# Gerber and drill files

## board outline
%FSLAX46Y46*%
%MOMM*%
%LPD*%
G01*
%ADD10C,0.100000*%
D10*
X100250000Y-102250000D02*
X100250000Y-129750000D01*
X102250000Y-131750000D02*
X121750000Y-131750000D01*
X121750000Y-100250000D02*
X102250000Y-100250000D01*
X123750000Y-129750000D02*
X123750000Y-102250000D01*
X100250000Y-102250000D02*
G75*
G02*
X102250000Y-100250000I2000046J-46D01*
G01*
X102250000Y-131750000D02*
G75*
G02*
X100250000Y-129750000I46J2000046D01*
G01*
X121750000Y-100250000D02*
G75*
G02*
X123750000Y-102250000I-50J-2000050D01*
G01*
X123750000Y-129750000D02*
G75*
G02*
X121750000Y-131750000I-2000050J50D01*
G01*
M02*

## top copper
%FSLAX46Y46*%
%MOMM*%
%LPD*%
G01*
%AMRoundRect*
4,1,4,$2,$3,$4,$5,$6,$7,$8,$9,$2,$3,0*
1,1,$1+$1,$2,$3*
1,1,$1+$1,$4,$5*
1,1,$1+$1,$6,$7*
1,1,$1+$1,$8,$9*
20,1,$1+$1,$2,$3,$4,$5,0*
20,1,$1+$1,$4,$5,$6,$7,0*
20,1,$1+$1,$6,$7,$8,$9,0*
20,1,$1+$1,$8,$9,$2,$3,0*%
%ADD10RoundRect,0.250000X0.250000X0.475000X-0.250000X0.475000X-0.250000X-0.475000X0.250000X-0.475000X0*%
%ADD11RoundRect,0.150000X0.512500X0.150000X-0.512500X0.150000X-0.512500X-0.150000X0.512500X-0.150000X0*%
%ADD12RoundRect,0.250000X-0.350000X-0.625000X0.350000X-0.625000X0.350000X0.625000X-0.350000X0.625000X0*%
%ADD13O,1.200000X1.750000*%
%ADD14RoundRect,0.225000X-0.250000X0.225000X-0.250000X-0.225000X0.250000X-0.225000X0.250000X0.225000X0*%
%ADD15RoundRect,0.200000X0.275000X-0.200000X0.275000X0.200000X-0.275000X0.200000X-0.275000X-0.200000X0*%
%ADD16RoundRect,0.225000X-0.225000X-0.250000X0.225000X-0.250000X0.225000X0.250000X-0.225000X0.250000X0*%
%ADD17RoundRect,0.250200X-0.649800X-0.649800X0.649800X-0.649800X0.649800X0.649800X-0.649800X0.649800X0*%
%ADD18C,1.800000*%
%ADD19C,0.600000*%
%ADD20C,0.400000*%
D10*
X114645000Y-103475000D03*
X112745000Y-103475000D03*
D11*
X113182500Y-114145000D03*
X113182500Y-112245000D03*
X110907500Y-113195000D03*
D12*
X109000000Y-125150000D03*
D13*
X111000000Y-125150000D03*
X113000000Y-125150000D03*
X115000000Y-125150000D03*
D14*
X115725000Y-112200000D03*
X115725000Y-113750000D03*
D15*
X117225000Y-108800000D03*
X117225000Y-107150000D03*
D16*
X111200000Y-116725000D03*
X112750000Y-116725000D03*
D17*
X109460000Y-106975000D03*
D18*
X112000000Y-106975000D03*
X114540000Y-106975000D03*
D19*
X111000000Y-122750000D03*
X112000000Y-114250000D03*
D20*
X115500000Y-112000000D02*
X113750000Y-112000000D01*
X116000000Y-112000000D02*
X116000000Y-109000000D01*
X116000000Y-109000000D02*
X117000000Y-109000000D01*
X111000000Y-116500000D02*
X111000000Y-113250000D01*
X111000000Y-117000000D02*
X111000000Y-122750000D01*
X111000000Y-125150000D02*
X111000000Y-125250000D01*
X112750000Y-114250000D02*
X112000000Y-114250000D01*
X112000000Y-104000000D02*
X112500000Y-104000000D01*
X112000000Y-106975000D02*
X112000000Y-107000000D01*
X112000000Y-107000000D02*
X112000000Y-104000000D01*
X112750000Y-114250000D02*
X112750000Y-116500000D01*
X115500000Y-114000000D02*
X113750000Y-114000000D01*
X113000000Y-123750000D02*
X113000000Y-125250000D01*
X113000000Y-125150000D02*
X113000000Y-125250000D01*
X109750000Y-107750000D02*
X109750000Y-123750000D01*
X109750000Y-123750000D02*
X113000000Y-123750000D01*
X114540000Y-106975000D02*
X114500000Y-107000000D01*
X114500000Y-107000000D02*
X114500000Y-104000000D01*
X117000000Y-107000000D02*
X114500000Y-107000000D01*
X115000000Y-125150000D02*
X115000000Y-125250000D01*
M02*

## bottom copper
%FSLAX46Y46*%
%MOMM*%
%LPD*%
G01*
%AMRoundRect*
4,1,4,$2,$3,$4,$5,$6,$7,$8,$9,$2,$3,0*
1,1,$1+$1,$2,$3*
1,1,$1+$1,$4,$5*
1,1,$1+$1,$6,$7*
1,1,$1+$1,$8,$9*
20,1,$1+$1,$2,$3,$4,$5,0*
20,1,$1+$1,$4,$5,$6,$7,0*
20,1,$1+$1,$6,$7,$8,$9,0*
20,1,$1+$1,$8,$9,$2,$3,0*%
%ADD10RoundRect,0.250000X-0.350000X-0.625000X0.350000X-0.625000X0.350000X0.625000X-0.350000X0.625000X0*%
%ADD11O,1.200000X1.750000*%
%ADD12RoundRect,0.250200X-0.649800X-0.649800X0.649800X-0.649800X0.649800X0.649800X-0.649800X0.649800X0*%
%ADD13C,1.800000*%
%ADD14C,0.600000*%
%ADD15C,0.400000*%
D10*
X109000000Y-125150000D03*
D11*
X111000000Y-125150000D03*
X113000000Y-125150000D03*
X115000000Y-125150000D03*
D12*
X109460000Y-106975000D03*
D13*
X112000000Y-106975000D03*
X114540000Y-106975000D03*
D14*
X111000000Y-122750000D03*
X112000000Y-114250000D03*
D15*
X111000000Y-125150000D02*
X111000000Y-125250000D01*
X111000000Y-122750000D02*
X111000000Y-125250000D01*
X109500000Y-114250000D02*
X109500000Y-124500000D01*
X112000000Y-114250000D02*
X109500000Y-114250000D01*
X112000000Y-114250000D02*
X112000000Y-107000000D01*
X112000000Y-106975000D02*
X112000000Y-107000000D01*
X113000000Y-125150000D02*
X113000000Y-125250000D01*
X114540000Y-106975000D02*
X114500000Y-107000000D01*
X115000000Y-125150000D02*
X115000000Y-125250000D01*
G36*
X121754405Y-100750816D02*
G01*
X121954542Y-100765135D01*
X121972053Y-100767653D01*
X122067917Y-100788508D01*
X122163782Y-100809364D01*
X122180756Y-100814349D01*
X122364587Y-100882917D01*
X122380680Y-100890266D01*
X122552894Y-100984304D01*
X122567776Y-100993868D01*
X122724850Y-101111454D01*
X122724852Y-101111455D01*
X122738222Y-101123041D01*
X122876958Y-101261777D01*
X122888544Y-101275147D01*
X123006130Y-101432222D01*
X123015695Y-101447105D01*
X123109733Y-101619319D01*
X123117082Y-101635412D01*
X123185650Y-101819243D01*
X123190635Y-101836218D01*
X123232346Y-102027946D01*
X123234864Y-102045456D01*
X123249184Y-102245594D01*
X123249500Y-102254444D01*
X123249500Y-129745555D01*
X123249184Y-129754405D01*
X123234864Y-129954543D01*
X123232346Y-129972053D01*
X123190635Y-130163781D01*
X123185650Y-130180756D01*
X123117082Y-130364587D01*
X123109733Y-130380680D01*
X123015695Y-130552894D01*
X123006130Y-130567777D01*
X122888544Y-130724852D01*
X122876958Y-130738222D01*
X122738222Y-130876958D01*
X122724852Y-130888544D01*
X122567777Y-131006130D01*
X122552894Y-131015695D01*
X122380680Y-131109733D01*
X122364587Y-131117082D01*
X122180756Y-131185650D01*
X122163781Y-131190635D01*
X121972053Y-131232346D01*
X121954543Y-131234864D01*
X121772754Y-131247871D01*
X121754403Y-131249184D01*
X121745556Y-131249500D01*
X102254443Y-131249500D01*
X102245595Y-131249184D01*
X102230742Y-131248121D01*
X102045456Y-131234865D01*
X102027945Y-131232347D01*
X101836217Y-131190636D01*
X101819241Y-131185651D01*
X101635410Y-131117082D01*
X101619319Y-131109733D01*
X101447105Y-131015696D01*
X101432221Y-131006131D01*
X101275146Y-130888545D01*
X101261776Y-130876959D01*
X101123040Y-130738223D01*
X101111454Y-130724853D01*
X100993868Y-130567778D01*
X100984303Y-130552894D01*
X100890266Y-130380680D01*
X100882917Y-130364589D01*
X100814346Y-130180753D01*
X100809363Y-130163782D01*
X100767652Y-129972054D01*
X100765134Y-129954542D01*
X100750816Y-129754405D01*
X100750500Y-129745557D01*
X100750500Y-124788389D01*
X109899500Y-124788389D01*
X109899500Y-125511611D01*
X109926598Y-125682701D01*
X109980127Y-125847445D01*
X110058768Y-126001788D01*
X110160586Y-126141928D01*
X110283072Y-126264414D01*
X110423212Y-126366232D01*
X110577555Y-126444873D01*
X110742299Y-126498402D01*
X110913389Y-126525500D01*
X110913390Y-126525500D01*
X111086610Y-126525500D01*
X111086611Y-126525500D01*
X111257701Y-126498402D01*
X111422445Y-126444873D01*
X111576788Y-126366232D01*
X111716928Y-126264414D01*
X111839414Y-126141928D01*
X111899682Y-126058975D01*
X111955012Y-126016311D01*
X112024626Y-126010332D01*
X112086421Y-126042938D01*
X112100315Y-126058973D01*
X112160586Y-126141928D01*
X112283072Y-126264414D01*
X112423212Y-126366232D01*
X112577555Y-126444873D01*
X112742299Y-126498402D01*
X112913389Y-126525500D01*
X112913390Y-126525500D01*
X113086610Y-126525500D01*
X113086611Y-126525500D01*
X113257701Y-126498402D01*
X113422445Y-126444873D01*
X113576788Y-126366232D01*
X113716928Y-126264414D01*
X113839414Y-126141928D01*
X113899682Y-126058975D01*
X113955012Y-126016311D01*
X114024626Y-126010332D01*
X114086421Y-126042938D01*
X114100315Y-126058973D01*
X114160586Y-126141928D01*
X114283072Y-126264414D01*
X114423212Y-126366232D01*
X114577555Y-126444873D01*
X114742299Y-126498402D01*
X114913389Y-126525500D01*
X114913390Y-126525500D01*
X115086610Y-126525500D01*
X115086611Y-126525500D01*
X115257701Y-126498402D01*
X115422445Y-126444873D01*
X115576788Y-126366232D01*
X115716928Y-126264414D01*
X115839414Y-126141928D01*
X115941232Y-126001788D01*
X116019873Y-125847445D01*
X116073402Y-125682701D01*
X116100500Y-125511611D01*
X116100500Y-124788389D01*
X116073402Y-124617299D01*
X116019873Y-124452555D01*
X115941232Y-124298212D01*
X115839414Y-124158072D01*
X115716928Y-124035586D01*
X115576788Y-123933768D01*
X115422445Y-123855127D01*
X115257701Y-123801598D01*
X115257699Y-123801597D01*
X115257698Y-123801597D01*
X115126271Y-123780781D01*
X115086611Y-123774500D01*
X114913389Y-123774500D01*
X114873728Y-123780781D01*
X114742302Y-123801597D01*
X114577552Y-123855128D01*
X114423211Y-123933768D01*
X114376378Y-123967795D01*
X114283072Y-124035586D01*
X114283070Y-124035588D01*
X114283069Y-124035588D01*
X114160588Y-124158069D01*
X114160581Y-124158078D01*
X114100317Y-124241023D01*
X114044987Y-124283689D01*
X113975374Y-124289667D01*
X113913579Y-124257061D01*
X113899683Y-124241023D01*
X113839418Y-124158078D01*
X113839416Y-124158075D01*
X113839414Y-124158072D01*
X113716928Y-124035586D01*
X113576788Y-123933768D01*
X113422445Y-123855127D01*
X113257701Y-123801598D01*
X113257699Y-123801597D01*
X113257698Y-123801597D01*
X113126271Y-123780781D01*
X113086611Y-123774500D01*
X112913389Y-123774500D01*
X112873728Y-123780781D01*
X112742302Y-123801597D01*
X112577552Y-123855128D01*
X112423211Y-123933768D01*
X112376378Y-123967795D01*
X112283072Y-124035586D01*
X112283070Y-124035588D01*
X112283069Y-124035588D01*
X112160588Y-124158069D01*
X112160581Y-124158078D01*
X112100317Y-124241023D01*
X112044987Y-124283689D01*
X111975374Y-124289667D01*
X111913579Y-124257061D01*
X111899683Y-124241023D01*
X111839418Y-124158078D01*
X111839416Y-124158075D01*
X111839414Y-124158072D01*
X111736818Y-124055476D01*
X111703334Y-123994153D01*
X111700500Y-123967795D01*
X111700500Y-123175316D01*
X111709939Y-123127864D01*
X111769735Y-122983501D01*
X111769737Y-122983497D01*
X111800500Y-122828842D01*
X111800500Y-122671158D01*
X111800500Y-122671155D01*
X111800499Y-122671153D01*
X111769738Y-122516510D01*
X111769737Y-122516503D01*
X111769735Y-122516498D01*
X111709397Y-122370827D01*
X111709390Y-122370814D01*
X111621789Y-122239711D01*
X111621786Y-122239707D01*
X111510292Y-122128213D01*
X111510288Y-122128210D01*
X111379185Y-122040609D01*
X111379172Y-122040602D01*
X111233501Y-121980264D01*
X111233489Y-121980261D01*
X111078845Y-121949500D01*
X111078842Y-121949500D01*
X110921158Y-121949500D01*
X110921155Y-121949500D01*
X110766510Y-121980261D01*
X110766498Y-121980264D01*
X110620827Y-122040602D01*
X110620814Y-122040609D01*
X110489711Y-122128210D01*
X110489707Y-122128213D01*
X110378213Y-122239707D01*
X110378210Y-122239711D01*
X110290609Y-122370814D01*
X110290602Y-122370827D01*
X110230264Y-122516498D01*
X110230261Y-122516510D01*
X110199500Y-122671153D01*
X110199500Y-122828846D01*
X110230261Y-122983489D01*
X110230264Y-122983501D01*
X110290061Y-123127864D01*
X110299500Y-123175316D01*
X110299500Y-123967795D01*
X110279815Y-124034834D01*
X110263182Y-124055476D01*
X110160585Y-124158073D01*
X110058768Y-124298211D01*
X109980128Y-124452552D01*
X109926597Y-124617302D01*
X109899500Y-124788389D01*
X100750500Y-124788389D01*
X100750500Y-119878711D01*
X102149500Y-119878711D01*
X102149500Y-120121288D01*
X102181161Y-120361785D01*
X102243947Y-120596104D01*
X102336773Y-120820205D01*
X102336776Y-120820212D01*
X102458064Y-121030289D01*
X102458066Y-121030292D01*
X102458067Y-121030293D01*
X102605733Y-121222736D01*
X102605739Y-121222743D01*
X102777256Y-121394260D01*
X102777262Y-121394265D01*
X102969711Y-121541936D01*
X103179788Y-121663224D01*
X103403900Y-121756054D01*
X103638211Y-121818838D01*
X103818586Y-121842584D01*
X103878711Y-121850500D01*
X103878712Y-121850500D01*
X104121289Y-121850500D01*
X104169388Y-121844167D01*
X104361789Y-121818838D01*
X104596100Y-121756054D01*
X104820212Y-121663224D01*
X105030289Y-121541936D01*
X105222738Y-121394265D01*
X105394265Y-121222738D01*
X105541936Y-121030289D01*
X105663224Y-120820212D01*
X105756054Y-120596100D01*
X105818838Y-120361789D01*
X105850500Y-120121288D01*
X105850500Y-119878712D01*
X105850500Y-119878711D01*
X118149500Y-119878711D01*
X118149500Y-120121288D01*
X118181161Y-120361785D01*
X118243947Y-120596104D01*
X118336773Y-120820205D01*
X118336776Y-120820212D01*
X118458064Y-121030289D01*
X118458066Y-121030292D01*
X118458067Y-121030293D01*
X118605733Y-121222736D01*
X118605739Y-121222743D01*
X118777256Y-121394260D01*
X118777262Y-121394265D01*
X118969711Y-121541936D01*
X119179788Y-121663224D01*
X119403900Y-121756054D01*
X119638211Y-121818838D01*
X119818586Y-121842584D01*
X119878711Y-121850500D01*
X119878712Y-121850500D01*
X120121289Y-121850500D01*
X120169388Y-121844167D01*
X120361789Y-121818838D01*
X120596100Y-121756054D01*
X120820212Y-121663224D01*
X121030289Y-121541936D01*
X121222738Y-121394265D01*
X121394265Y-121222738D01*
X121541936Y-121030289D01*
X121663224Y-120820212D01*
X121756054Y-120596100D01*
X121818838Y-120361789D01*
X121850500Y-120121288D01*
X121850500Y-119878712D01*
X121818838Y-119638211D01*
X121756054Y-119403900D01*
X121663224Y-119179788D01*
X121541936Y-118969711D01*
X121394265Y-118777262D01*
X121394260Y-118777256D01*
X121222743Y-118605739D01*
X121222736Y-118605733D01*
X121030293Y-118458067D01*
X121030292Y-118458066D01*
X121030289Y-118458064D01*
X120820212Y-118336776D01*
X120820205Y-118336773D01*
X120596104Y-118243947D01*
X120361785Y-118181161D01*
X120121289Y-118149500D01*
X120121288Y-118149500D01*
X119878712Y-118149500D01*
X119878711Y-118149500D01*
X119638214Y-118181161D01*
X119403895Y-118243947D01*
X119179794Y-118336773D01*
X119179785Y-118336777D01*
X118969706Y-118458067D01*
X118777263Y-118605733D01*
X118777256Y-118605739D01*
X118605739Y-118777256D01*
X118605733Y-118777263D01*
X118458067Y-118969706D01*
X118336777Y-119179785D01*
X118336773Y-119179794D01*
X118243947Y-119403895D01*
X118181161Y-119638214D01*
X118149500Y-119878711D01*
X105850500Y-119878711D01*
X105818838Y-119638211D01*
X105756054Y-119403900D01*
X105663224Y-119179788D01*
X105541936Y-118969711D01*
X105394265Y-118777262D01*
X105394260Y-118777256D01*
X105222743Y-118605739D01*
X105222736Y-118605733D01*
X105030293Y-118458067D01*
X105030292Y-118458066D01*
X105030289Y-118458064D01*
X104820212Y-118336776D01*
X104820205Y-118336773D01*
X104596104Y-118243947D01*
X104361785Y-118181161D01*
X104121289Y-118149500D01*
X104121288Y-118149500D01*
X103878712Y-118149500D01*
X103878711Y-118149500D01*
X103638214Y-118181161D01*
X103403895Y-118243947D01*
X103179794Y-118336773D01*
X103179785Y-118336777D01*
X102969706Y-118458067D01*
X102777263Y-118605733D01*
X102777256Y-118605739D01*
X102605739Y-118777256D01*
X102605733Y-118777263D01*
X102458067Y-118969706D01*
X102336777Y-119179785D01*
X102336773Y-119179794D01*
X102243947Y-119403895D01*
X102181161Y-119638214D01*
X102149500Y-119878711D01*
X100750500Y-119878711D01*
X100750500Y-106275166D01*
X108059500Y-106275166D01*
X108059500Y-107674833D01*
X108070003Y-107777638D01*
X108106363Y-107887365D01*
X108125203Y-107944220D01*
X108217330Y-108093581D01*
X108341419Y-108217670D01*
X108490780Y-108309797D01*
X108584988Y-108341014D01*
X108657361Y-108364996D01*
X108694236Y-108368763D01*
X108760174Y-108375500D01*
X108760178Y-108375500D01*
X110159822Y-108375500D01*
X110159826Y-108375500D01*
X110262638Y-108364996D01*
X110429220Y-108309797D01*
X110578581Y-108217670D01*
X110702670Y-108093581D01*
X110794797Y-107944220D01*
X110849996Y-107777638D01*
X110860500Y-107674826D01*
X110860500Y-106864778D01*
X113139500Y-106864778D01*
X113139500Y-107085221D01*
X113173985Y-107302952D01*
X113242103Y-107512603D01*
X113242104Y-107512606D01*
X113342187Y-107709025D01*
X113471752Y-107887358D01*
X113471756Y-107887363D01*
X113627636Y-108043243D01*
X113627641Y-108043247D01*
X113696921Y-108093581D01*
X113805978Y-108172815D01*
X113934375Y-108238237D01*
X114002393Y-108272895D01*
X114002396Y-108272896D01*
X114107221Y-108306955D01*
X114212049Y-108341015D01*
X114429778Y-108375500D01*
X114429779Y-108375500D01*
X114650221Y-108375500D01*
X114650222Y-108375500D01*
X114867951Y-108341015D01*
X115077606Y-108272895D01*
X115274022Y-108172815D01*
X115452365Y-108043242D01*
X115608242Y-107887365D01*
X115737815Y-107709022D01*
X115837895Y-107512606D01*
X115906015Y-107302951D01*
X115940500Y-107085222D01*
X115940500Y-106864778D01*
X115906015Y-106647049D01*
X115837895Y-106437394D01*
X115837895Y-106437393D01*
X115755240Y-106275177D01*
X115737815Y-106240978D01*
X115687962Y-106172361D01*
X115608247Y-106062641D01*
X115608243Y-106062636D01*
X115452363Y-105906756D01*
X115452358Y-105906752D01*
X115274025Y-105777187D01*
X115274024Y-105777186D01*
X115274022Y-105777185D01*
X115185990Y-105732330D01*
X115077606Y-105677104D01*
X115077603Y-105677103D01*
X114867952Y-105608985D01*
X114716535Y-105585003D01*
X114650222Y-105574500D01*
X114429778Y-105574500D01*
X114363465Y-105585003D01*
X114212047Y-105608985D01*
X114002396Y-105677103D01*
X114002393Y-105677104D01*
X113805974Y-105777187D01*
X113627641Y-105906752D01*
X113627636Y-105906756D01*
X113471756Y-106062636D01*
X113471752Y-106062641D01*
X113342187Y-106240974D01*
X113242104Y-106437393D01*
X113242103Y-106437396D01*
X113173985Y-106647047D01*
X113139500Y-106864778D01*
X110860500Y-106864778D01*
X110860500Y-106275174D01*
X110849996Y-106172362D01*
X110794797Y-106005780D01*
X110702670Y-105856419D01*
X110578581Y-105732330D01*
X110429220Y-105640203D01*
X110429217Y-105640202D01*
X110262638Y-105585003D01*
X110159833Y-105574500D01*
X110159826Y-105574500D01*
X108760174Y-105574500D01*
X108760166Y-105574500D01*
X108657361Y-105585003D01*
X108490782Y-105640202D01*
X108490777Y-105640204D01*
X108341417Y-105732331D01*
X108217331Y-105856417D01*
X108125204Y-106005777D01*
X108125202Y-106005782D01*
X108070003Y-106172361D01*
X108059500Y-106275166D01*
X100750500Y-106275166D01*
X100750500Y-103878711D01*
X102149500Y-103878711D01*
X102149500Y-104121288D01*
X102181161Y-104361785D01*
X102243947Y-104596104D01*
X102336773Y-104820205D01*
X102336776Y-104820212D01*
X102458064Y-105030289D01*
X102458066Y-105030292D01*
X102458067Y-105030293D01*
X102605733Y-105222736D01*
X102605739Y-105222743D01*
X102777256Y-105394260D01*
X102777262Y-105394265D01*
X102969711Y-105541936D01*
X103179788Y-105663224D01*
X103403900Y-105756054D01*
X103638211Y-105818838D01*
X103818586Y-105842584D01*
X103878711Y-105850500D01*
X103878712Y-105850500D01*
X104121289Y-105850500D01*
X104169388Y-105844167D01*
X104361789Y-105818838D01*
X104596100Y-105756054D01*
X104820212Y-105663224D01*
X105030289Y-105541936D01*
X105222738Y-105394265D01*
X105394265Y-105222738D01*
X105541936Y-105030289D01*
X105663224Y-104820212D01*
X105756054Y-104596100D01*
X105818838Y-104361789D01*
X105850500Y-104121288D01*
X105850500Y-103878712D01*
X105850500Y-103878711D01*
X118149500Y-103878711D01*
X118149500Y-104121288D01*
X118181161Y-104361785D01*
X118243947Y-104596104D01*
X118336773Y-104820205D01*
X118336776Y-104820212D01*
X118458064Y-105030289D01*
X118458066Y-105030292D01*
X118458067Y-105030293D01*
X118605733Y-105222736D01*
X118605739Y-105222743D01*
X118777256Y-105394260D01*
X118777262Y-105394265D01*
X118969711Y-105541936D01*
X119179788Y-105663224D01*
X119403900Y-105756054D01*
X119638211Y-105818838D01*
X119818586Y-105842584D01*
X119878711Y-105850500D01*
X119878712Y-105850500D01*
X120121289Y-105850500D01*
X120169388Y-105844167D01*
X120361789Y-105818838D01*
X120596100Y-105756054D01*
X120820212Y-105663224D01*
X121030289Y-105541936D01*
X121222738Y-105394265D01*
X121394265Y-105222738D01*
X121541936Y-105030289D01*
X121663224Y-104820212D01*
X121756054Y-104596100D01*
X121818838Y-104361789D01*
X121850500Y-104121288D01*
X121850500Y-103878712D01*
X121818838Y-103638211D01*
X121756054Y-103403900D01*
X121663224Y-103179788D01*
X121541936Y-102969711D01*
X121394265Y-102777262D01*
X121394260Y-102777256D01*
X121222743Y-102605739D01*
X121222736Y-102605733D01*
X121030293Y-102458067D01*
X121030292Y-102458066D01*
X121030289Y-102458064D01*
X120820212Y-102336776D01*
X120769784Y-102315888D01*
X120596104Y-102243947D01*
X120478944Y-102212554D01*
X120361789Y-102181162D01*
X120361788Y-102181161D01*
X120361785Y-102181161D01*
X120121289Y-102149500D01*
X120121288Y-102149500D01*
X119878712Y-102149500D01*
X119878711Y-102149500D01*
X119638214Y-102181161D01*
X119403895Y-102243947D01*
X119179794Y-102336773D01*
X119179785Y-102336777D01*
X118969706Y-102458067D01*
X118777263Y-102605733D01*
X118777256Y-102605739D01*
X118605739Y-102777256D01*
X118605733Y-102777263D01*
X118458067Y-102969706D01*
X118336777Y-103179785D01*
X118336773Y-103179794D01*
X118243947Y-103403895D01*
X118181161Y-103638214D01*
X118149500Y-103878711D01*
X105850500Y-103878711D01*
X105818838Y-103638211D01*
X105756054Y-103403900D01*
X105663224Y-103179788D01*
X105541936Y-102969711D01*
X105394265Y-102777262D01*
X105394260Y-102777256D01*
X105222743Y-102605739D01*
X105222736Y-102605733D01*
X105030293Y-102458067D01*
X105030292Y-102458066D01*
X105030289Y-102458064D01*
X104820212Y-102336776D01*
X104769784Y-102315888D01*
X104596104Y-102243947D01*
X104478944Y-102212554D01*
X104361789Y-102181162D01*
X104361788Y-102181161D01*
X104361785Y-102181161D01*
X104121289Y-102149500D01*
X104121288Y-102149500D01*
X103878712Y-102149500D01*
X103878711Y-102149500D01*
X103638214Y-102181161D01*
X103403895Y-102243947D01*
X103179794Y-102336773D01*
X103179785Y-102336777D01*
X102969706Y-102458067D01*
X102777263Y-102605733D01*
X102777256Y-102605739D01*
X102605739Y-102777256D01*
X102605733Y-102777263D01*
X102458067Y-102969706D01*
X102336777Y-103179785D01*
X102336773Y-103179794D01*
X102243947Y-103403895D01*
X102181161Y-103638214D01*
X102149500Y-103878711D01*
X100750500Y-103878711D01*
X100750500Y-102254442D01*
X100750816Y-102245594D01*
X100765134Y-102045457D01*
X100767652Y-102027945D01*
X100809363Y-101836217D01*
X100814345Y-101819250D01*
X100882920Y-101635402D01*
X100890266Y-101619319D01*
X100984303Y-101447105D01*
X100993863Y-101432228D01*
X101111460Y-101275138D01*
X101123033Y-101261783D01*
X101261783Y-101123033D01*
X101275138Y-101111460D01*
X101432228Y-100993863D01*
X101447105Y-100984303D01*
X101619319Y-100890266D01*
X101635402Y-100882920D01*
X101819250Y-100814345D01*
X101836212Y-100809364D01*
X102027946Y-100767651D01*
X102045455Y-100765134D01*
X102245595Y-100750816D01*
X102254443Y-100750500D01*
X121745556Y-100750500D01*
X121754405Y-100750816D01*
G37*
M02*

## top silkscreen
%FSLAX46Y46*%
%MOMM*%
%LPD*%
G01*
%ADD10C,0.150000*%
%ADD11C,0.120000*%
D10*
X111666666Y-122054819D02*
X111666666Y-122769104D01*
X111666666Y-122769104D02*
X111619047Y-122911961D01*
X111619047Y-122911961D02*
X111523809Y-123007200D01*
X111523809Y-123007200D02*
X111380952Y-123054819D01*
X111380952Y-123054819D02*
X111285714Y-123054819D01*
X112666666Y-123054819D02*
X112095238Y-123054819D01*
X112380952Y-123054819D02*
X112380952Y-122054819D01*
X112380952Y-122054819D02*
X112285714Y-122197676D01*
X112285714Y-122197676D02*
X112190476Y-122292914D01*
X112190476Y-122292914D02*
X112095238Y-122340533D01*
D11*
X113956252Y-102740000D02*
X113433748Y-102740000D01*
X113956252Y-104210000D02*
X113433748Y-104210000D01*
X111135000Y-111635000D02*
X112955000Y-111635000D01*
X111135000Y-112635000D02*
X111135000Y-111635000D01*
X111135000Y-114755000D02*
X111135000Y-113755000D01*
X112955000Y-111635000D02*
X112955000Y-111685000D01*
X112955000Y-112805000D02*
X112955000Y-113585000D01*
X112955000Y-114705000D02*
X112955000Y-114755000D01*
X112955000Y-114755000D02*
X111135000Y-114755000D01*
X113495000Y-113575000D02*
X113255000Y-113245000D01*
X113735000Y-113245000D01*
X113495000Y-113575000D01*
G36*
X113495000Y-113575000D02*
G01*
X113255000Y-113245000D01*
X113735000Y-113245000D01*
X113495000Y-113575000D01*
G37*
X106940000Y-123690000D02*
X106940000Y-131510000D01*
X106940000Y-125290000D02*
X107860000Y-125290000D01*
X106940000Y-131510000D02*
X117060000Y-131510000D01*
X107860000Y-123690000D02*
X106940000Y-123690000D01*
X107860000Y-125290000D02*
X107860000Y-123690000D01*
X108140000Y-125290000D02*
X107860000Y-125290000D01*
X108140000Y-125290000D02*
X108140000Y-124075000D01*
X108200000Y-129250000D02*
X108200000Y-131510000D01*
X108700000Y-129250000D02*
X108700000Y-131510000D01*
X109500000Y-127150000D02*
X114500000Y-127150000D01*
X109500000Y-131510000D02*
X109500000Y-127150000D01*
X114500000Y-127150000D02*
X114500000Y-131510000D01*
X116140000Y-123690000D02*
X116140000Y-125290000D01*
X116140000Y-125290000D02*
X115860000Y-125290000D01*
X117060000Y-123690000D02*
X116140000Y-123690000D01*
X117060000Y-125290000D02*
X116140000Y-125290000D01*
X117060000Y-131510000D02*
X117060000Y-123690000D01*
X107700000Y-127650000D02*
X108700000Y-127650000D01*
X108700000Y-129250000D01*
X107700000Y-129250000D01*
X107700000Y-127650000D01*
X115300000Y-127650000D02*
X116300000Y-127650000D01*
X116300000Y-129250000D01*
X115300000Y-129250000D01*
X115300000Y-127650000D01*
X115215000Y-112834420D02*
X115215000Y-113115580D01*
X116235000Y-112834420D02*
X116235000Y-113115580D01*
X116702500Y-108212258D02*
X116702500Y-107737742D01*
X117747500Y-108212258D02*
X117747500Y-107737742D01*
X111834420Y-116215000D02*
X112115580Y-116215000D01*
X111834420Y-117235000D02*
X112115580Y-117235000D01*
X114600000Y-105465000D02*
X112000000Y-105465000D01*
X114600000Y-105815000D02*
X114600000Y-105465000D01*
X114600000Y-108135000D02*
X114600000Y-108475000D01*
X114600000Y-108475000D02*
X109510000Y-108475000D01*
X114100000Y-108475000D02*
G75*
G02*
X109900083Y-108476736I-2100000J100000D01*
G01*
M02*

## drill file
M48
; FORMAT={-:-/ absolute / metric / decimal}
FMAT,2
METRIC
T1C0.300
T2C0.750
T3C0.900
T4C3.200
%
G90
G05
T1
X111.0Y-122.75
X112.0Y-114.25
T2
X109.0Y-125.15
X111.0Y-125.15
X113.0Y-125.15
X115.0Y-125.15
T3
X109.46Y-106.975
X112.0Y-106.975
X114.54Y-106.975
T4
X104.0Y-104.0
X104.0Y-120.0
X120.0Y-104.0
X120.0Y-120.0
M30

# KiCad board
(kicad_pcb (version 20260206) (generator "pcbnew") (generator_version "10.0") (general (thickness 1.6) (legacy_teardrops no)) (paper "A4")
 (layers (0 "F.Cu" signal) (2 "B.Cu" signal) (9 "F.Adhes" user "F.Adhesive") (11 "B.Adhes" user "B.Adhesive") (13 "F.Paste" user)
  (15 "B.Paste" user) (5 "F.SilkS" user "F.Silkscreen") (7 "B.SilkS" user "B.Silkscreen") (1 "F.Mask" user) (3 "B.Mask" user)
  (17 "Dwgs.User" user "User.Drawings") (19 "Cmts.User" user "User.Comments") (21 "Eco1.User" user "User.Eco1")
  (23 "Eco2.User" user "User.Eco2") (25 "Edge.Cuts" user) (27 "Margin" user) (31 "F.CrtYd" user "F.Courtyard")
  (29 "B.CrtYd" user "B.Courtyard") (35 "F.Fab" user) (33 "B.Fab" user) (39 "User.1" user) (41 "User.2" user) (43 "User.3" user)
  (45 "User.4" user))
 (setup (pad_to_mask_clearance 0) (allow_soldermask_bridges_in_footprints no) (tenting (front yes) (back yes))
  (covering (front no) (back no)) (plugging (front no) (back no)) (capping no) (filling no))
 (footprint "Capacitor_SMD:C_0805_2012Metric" (layer "F.Cu") (at 113.695 103.475 180)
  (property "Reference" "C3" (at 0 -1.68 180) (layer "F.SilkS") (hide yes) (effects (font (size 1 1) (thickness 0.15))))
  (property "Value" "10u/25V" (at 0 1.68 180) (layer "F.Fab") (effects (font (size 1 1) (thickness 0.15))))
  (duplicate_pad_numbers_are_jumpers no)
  (fp_line (start -0.261252 0.735) (end 0.261252 0.735) (stroke (width 0.12) (type solid)) (layer "F.SilkS"))
  (fp_line (start -0.261252 -0.735) (end 0.261252 -0.735) (stroke (width 0.12) (type solid)) (layer "F.SilkS"))
  (pad "1" smd roundrect (at -0.95 0 180) (size 1 1.45) (layers "F.Cu" "F.Mask" "F.Paste") (roundrect_rratio 0.25) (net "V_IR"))
  (pad "2" smd roundrect (at 0.95 0 180) (size 1 1.45) (layers "F.Cu" "F.Mask" "F.Paste") (roundrect_rratio 0.25) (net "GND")))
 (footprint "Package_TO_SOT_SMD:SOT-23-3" (layer "F.Cu") (at 112.045 113.195 180)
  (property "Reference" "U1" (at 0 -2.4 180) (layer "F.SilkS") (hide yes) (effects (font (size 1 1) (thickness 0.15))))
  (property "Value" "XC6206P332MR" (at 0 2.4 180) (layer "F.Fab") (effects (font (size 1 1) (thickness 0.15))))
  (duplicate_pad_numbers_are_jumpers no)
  (fp_line (start 0.91 1.56) (end -0.91 1.56) (stroke (width 0.12) (type solid)) (layer "F.SilkS"))
  (fp_line (start 0.91 0.56) (end 0.91 1.56) (stroke (width 0.12) (type solid)) (layer "F.SilkS"))
  (fp_line (start 0.91 -1.56) (end 0.91 -0.56) (stroke (width 0.12) (type solid)) (layer "F.SilkS"))
  (fp_line (start -0.91 1.56) (end -0.91 1.51) (stroke (width 0.12) (type solid)) (layer "F.SilkS"))
  (fp_line (start -0.91 0.39) (end -0.91 -0.39) (stroke (width 0.12) (type solid)) (layer "F.SilkS"))
  (fp_line (start -0.91 -1.51) (end -0.91 -1.56) (stroke (width 0.12) (type solid)) (layer "F.SilkS"))
  (fp_line (start -0.91 -1.56) (end 0.91 -1.56) (stroke (width 0.12) (type solid)) (layer "F.SilkS"))
  (fp_poly (pts (xy -1.45 -0.38) (xy -1.21 -0.05) (xy -1.69 -0.05)) (stroke (width 0.12) (type solid)) (fill yes) (layer "F.SilkS"))
  (pad "1" smd roundrect (at -1.1375 -0.95 180) (size 1.325 0.6) (layers "F.Cu" "F.Mask" "F.Paste") (roundrect_rratio 0.25) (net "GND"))
  (pad "2" smd roundrect (at -1.1375 0.95 180) (size 1.325 0.6) (layers "F.Cu" "F.Mask" "F.Paste") (roundrect_rratio 0.25) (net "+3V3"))
  (pad "3" smd roundrect (at 1.1375 0 180) (size 1.325 0.6) (layers "F.Cu" "F.Mask" "F.Paste") (roundrect_rratio 0.25) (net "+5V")))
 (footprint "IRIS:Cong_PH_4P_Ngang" (layer "F.Cu") (at 109 125.15)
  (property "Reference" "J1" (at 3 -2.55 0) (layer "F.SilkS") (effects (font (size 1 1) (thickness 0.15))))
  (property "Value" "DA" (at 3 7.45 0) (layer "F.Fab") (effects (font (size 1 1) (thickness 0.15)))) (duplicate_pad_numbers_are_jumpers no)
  (fp_line (start -2.06 -1.46) (end -2.06 6.36) (stroke (width 0.12) (type solid)) (layer "F.SilkS"))
  (fp_line (start -2.06 0.14) (end -1.14 0.14) (stroke (width 0.12) (type solid)) (layer "F.SilkS"))
  (fp_line (start -2.06 6.36) (end 8.06 6.36) (stroke (width 0.12) (type solid)) (layer "F.SilkS"))
  (fp_line (start -1.14 -1.46) (end -2.06 -1.46) (stroke (width 0.12) (type solid)) (layer "F.SilkS"))
  (fp_line (start -1.14 0.14) (end -1.14 -1.46) (stroke (width 0.12) (type solid)) (layer "F.SilkS"))
  (fp_line (start -0.86 0.14) (end -1.14 0.14) (stroke (width 0.12) (type solid)) (layer "F.SilkS"))
  (fp_line (start -0.86 0.14) (end -0.86 -1.075) (stroke (width 0.12) (type solid)) (layer "F.SilkS"))
  (fp_line (start -0.8 4.1) (end -0.8 6.36) (stroke (width 0.12) (type solid)) (layer "F.SilkS"))
  (fp_line (start -0.3 4.1) (end -0.3 6.36) (stroke (width 0.12) (type solid)) (layer "F.SilkS"))
  (fp_line (start 0.5 2) (end 5.5 2) (stroke (width 0.12) (type solid)) (layer "F.SilkS"))
  (fp_line (start 0.5 6.36) (end 0.5 2) (stroke (width 0.12) (type solid)) (layer "F.SilkS"))
  (fp_line (start 5.5 2) (end 5.5 6.36) (stroke (width 0.12) (type solid)) (layer "F.SilkS"))
  (fp_line (start 7.14 -1.46) (end 7.14 0.14) (stroke (width 0.12) (type solid)) (layer "F.SilkS"))
  (fp_line (start 7.14 0.14) (end 6.86 0.14) (stroke (width 0.12) (type solid)) (layer "F.SilkS"))
  (fp_line (start 8.06 -1.46) (end 7.14 -1.46) (stroke (width 0.12) (type solid)) (layer "F.SilkS"))
  (fp_line (start 8.06 0.14) (end 7.14 0.14) (stroke (width 0.12) (type solid)) (layer "F.SilkS"))
  (fp_line (start 8.06 6.36) (end 8.06 -1.46) (stroke (width 0.12) (type solid)) (layer "F.SilkS"))
  (fp_rect (start -1.3 2.5) (end -0.3 4.1) (stroke (width 0.12) (type solid)) (fill no) (layer "F.SilkS"))
  (fp_rect (start 6.3 2.5) (end 7.3 4.1) (stroke (width 0.12) (type solid)) (fill no) (layer "F.SilkS"))
  (pad "1" thru_hole roundrect (at 0 0) (size 1.2 1.75) (drill 0.75) (layers "*.Cu" "*.Mask") (remove_unused_layers no)
   (roundrect_rratio 0.208333) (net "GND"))
  (pad "2" thru_hole oval (at 2 0) (size 1.2 1.75) (drill 0.75) (layers "*.Cu" "*.Mask") (remove_unused_layers no) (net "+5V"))
  (pad "3" thru_hole oval (at 4 0) (size 1.2 1.75) (drill 0.75) (layers "*.Cu" "*.Mask") (remove_unused_layers no) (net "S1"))
  (pad "4" thru_hole oval (at 6 0) (size 1.2 1.75) (drill 0.75) (layers "*.Cu" "*.Mask") (remove_unused_layers no)
   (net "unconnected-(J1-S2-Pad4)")))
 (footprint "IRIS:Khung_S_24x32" (layer "F.Cu") (at 100 132)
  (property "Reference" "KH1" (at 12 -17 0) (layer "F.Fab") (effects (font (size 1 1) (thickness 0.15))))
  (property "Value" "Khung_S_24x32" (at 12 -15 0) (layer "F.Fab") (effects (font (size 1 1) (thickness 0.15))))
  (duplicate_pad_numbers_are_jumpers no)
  (fp_line (start 0.25 -29.75) (end 0.25 -2.25) (stroke (width 0.1) (type solid)) (layer "Edge.Cuts"))
  (fp_line (start 2.25 -0.25) (end 21.75 -0.25) (stroke (width 0.1) (type solid)) (layer "Edge.Cuts"))
  (fp_line (start 21.75 -31.75) (end 2.25 -31.75) (stroke (width 0.1) (type solid)) (layer "Edge.Cuts"))
  (fp_line (start 23.75 -2.25) (end 23.75 -29.75) (stroke (width 0.1) (type solid)) (layer "Edge.Cuts"))
  (fp_arc (start 0.25 -29.75) (mid 0.8358 -31.1642) (end 2.25 -31.75) (stroke (width 0.1) (type solid)) (layer "Edge.Cuts"))
  (fp_arc (start 2.25 -0.25) (mid 0.8358 -0.8358) (end 0.25 -2.25) (stroke (width 0.1) (type solid)) (layer "Edge.Cuts"))
  (fp_arc (start 21.75 -31.75) (mid 23.164199 -31.164199) (end 23.75 -29.75) (stroke (width 0.1) (type solid)) (layer "Edge.Cuts"))
  (fp_arc (start 23.75 -2.25) (mid 23.164199 -0.835801) (end 21.75 -0.25) (stroke (width 0.1) (type solid)) (layer "Edge.Cuts"))
  (pad "" np_thru_hole circle (at 4 -28) (size 3.2 3.2) (drill 3.2) (layers "*.Cu" "*.Mask"))
  (pad "" np_thru_hole circle (at 4 -12) (size 3.2 3.2) (drill 3.2) (layers "*.Cu" "*.Mask"))
  (pad "" np_thru_hole circle (at 20 -28) (size 3.2 3.2) (drill 3.2) (layers "*.Cu" "*.Mask"))
  (pad "" np_thru_hole circle (at 20 -12) (size 3.2 3.2) (drill 3.2) (layers "*.Cu" "*.Mask")))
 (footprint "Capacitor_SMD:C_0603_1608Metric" (layer "F.Cu") (at 115.725 112.975 -90)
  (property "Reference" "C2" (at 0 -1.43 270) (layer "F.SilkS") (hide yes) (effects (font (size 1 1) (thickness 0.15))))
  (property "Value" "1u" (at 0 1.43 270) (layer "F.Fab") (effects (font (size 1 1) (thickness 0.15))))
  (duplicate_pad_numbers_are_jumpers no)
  (fp_line (start -0.14058 0.51) (end 0.14058 0.51) (stroke (width 0.12) (type solid)) (layer "F.SilkS"))
  (fp_line (start -0.14058 -0.51) (end 0.14058 -0.51) (stroke (width 0.12) (type solid)) (layer "F.SilkS"))
  (pad "1" smd roundrect (at -0.775 0 270) (size 0.9 0.95) (layers "F.Cu" "F.Mask" "F.Paste") (roundrect_rratio 0.25) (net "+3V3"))
  (pad "2" smd roundrect (at 0.775 0 270) (size 0.9 0.95) (layers "F.Cu" "F.Mask" "F.Paste") (roundrect_rratio 0.25) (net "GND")))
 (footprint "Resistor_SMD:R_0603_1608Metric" (layer "F.Cu") (at 117.225 107.975 90)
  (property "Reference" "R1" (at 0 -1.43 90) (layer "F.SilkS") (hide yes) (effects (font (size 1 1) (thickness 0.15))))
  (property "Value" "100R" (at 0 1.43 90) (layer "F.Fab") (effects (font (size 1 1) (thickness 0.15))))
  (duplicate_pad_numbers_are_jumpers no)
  (fp_line (start -0.237258 -0.5225) (end 0.237258 -0.5225) (stroke (width 0.12) (type solid)) (layer "F.SilkS"))
  (fp_line (start -0.237258 0.5225) (end 0.237258 0.5225) (stroke (width 0.12) (type solid)) (layer "F.SilkS"))
  (pad "1" smd roundrect (at -0.825 0 90) (size 0.8 0.95) (layers "F.Cu" "F.Mask" "F.Paste") (roundrect_rratio 0.25) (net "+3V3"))
  (pad "2" smd roundrect (at 0.825 0 90) (size 0.8 0.95) (layers "F.Cu" "F.Mask" "F.Paste") (roundrect_rratio 0.25) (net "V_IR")))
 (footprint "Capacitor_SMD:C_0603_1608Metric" (layer "F.Cu") (at 111.975 116.725)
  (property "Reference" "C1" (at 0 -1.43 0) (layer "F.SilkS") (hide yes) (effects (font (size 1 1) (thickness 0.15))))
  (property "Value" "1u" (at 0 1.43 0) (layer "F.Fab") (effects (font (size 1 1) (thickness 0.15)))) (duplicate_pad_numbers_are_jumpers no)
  (fp_line (start -0.14058 -0.51) (end 0.14058 -0.51) (stroke (width 0.12) (type solid)) (layer "F.SilkS"))
  (fp_line (start -0.14058 0.51) (end 0.14058 0.51) (stroke (width 0.12) (type solid)) (layer "F.SilkS"))
  (pad "1" smd roundrect (at -0.775 0) (size 0.9 0.95) (layers "F.Cu" "F.Mask" "F.Paste") (roundrect_rratio 0.25) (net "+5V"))
  (pad "2" smd roundrect (at 0.775 0) (size 0.9 0.95) (layers "F.Cu" "F.Mask" "F.Paste") (roundrect_rratio 0.25) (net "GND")))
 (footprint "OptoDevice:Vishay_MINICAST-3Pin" (layer "F.Cu") (at 109.46 106.975)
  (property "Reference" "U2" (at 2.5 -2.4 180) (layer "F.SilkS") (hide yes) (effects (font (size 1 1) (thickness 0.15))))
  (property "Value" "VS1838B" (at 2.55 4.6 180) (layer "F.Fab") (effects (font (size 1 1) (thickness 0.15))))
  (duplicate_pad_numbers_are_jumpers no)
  (fp_line (start 5.14 -1.51) (end 2.54 -1.51) (stroke (width 0.12) (type solid)) (layer "F.SilkS"))
  (fp_line (start 5.14 -1.16) (end 5.14 -1.51) (stroke (width 0.12) (type solid)) (layer "F.SilkS"))
  (fp_line (start 5.14 1.16) (end 5.14 1.5) (stroke (width 0.12) (type solid)) (layer "F.SilkS"))
  (fp_line (start 5.14 1.5) (end 0.05 1.5) (stroke (width 0.12) (type solid)) (layer "F.SilkS"))
  (fp_arc (start 4.64 1.5) (mid 2.540869 3.502379) (end 0.440083 1.501736) (stroke (width 0.12) (type solid)) (layer "F.SilkS"))
  (pad "1" thru_hole roundrect (at 0 0) (size 1.8 1.8) (drill 0.9) (layers "*.Cu" "*.Mask") (remove_unused_layers no)
   (roundrect_rratio 0.139) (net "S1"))
  (pad "2" thru_hole circle (at 2.54 0) (size 1.8 1.8) (drill 0.9) (layers "*.Cu" "*.Mask") (remove_unused_layers no) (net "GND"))
  (pad "3" thru_hole circle (at 5.08 0) (size 1.8 1.8) (drill 0.9) (layers "*.Cu" "*.Mask") (remove_unused_layers no) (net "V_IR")))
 (segment (start 115.5 112) (end 113.75 112) (width 0.4) (layer "F.Cu") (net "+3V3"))
 (segment (start 116 112) (end 116 109) (width 0.4) (layer "F.Cu") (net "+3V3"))
 (segment (start 116 109) (end 117 109) (width 0.4) (layer "F.Cu") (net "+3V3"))
 (segment (start 111 116.5) (end 111 113.25) (width 0.4) (layer "F.Cu") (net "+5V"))
 (segment (start 111 117) (end 111 122.75) (width 0.4) (layer "F.Cu") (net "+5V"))
 (segment (start 111 125.15) (end 111 125.25) (width 0.4) (layer "F.Cu") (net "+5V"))
 (via (at 111 122.75) (size 0.6) (drill 0.3) (layers "F.Cu" "B.Cu") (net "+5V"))
 (segment (start 111 125.15) (end 111 125.25) (width 0.4) (layer "B.Cu") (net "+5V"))
 (segment (start 111 122.75) (end 111 125.25) (width 0.4) (layer "B.Cu") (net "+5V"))
 (segment (start 112.75 114.25) (end 112 114.25) (width 0.4) (layer "F.Cu") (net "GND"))
 (segment (start 112 104) (end 112.5 104) (width 0.4) (layer "F.Cu") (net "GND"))
 (segment (start 112 106.975) (end 112 107) (width 0.4) (layer "F.Cu") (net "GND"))
 (segment (start 112 107) (end 112 104) (width 0.4) (layer "F.Cu") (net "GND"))
 (segment (start 112.75 114.25) (end 112.75 116.5) (width 0.4) (layer "F.Cu") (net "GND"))
 (segment (start 115.5 114) (end 113.75 114) (width 0.4) (layer "F.Cu") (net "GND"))
 (via (at 112 114.25) (size 0.6) (drill 0.3) (layers "F.Cu" "B.Cu") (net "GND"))
 (segment (start 109.5 114.25) (end 109.5 124.5) (width 0.4) (layer "B.Cu") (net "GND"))
 (segment (start 112 114.25) (end 109.5 114.25) (width 0.4) (layer "B.Cu") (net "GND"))
 (segment (start 112 114.25) (end 112 107) (width 0.4) (layer "B.Cu") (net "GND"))
 (segment (start 112 106.975) (end 112 107) (width 0.4) (layer "B.Cu") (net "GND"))
 (segment (start 113 123.75) (end 113 125.25) (width 0.4) (layer "F.Cu") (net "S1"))
 (segment (start 113 125.15) (end 113 125.25) (width 0.4) (layer "F.Cu") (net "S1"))
 (segment (start 109.75 107.75) (end 109.75 123.75) (width 0.4) (layer "F.Cu") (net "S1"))
 (segment (start 109.75 123.75) (end 113 123.75) (width 0.4) (layer "F.Cu") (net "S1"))
 (segment (start 113 125.15) (end 113 125.25) (width 0.4) (layer "B.Cu") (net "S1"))
 (segment (start 114.54 106.975) (end 114.5 107) (width 0.4) (layer "F.Cu") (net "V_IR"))
 (segment (start 114.5 107) (end 114.5 104) (width 0.4) (layer "F.Cu") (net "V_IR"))
 (segment (start 117 107) (end 114.5 107) (width 0.4) (layer "F.Cu") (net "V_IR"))
 (segment (start 114.54 106.975) (end 114.5 107) (width 0.4) (layer "B.Cu") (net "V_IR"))
 (segment (start 115 125.15) (end 115 125.25) (width 0.4) (layer "F.Cu") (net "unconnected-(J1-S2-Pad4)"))
 (segment (start 115 125.15) (end 115 125.25) (width 0.4) (layer "B.Cu") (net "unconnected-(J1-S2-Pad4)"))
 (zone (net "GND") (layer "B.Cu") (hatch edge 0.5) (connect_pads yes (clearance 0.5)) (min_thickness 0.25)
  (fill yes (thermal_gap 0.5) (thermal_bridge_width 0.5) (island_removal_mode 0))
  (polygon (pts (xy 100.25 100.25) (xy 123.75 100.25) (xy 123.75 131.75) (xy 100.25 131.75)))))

